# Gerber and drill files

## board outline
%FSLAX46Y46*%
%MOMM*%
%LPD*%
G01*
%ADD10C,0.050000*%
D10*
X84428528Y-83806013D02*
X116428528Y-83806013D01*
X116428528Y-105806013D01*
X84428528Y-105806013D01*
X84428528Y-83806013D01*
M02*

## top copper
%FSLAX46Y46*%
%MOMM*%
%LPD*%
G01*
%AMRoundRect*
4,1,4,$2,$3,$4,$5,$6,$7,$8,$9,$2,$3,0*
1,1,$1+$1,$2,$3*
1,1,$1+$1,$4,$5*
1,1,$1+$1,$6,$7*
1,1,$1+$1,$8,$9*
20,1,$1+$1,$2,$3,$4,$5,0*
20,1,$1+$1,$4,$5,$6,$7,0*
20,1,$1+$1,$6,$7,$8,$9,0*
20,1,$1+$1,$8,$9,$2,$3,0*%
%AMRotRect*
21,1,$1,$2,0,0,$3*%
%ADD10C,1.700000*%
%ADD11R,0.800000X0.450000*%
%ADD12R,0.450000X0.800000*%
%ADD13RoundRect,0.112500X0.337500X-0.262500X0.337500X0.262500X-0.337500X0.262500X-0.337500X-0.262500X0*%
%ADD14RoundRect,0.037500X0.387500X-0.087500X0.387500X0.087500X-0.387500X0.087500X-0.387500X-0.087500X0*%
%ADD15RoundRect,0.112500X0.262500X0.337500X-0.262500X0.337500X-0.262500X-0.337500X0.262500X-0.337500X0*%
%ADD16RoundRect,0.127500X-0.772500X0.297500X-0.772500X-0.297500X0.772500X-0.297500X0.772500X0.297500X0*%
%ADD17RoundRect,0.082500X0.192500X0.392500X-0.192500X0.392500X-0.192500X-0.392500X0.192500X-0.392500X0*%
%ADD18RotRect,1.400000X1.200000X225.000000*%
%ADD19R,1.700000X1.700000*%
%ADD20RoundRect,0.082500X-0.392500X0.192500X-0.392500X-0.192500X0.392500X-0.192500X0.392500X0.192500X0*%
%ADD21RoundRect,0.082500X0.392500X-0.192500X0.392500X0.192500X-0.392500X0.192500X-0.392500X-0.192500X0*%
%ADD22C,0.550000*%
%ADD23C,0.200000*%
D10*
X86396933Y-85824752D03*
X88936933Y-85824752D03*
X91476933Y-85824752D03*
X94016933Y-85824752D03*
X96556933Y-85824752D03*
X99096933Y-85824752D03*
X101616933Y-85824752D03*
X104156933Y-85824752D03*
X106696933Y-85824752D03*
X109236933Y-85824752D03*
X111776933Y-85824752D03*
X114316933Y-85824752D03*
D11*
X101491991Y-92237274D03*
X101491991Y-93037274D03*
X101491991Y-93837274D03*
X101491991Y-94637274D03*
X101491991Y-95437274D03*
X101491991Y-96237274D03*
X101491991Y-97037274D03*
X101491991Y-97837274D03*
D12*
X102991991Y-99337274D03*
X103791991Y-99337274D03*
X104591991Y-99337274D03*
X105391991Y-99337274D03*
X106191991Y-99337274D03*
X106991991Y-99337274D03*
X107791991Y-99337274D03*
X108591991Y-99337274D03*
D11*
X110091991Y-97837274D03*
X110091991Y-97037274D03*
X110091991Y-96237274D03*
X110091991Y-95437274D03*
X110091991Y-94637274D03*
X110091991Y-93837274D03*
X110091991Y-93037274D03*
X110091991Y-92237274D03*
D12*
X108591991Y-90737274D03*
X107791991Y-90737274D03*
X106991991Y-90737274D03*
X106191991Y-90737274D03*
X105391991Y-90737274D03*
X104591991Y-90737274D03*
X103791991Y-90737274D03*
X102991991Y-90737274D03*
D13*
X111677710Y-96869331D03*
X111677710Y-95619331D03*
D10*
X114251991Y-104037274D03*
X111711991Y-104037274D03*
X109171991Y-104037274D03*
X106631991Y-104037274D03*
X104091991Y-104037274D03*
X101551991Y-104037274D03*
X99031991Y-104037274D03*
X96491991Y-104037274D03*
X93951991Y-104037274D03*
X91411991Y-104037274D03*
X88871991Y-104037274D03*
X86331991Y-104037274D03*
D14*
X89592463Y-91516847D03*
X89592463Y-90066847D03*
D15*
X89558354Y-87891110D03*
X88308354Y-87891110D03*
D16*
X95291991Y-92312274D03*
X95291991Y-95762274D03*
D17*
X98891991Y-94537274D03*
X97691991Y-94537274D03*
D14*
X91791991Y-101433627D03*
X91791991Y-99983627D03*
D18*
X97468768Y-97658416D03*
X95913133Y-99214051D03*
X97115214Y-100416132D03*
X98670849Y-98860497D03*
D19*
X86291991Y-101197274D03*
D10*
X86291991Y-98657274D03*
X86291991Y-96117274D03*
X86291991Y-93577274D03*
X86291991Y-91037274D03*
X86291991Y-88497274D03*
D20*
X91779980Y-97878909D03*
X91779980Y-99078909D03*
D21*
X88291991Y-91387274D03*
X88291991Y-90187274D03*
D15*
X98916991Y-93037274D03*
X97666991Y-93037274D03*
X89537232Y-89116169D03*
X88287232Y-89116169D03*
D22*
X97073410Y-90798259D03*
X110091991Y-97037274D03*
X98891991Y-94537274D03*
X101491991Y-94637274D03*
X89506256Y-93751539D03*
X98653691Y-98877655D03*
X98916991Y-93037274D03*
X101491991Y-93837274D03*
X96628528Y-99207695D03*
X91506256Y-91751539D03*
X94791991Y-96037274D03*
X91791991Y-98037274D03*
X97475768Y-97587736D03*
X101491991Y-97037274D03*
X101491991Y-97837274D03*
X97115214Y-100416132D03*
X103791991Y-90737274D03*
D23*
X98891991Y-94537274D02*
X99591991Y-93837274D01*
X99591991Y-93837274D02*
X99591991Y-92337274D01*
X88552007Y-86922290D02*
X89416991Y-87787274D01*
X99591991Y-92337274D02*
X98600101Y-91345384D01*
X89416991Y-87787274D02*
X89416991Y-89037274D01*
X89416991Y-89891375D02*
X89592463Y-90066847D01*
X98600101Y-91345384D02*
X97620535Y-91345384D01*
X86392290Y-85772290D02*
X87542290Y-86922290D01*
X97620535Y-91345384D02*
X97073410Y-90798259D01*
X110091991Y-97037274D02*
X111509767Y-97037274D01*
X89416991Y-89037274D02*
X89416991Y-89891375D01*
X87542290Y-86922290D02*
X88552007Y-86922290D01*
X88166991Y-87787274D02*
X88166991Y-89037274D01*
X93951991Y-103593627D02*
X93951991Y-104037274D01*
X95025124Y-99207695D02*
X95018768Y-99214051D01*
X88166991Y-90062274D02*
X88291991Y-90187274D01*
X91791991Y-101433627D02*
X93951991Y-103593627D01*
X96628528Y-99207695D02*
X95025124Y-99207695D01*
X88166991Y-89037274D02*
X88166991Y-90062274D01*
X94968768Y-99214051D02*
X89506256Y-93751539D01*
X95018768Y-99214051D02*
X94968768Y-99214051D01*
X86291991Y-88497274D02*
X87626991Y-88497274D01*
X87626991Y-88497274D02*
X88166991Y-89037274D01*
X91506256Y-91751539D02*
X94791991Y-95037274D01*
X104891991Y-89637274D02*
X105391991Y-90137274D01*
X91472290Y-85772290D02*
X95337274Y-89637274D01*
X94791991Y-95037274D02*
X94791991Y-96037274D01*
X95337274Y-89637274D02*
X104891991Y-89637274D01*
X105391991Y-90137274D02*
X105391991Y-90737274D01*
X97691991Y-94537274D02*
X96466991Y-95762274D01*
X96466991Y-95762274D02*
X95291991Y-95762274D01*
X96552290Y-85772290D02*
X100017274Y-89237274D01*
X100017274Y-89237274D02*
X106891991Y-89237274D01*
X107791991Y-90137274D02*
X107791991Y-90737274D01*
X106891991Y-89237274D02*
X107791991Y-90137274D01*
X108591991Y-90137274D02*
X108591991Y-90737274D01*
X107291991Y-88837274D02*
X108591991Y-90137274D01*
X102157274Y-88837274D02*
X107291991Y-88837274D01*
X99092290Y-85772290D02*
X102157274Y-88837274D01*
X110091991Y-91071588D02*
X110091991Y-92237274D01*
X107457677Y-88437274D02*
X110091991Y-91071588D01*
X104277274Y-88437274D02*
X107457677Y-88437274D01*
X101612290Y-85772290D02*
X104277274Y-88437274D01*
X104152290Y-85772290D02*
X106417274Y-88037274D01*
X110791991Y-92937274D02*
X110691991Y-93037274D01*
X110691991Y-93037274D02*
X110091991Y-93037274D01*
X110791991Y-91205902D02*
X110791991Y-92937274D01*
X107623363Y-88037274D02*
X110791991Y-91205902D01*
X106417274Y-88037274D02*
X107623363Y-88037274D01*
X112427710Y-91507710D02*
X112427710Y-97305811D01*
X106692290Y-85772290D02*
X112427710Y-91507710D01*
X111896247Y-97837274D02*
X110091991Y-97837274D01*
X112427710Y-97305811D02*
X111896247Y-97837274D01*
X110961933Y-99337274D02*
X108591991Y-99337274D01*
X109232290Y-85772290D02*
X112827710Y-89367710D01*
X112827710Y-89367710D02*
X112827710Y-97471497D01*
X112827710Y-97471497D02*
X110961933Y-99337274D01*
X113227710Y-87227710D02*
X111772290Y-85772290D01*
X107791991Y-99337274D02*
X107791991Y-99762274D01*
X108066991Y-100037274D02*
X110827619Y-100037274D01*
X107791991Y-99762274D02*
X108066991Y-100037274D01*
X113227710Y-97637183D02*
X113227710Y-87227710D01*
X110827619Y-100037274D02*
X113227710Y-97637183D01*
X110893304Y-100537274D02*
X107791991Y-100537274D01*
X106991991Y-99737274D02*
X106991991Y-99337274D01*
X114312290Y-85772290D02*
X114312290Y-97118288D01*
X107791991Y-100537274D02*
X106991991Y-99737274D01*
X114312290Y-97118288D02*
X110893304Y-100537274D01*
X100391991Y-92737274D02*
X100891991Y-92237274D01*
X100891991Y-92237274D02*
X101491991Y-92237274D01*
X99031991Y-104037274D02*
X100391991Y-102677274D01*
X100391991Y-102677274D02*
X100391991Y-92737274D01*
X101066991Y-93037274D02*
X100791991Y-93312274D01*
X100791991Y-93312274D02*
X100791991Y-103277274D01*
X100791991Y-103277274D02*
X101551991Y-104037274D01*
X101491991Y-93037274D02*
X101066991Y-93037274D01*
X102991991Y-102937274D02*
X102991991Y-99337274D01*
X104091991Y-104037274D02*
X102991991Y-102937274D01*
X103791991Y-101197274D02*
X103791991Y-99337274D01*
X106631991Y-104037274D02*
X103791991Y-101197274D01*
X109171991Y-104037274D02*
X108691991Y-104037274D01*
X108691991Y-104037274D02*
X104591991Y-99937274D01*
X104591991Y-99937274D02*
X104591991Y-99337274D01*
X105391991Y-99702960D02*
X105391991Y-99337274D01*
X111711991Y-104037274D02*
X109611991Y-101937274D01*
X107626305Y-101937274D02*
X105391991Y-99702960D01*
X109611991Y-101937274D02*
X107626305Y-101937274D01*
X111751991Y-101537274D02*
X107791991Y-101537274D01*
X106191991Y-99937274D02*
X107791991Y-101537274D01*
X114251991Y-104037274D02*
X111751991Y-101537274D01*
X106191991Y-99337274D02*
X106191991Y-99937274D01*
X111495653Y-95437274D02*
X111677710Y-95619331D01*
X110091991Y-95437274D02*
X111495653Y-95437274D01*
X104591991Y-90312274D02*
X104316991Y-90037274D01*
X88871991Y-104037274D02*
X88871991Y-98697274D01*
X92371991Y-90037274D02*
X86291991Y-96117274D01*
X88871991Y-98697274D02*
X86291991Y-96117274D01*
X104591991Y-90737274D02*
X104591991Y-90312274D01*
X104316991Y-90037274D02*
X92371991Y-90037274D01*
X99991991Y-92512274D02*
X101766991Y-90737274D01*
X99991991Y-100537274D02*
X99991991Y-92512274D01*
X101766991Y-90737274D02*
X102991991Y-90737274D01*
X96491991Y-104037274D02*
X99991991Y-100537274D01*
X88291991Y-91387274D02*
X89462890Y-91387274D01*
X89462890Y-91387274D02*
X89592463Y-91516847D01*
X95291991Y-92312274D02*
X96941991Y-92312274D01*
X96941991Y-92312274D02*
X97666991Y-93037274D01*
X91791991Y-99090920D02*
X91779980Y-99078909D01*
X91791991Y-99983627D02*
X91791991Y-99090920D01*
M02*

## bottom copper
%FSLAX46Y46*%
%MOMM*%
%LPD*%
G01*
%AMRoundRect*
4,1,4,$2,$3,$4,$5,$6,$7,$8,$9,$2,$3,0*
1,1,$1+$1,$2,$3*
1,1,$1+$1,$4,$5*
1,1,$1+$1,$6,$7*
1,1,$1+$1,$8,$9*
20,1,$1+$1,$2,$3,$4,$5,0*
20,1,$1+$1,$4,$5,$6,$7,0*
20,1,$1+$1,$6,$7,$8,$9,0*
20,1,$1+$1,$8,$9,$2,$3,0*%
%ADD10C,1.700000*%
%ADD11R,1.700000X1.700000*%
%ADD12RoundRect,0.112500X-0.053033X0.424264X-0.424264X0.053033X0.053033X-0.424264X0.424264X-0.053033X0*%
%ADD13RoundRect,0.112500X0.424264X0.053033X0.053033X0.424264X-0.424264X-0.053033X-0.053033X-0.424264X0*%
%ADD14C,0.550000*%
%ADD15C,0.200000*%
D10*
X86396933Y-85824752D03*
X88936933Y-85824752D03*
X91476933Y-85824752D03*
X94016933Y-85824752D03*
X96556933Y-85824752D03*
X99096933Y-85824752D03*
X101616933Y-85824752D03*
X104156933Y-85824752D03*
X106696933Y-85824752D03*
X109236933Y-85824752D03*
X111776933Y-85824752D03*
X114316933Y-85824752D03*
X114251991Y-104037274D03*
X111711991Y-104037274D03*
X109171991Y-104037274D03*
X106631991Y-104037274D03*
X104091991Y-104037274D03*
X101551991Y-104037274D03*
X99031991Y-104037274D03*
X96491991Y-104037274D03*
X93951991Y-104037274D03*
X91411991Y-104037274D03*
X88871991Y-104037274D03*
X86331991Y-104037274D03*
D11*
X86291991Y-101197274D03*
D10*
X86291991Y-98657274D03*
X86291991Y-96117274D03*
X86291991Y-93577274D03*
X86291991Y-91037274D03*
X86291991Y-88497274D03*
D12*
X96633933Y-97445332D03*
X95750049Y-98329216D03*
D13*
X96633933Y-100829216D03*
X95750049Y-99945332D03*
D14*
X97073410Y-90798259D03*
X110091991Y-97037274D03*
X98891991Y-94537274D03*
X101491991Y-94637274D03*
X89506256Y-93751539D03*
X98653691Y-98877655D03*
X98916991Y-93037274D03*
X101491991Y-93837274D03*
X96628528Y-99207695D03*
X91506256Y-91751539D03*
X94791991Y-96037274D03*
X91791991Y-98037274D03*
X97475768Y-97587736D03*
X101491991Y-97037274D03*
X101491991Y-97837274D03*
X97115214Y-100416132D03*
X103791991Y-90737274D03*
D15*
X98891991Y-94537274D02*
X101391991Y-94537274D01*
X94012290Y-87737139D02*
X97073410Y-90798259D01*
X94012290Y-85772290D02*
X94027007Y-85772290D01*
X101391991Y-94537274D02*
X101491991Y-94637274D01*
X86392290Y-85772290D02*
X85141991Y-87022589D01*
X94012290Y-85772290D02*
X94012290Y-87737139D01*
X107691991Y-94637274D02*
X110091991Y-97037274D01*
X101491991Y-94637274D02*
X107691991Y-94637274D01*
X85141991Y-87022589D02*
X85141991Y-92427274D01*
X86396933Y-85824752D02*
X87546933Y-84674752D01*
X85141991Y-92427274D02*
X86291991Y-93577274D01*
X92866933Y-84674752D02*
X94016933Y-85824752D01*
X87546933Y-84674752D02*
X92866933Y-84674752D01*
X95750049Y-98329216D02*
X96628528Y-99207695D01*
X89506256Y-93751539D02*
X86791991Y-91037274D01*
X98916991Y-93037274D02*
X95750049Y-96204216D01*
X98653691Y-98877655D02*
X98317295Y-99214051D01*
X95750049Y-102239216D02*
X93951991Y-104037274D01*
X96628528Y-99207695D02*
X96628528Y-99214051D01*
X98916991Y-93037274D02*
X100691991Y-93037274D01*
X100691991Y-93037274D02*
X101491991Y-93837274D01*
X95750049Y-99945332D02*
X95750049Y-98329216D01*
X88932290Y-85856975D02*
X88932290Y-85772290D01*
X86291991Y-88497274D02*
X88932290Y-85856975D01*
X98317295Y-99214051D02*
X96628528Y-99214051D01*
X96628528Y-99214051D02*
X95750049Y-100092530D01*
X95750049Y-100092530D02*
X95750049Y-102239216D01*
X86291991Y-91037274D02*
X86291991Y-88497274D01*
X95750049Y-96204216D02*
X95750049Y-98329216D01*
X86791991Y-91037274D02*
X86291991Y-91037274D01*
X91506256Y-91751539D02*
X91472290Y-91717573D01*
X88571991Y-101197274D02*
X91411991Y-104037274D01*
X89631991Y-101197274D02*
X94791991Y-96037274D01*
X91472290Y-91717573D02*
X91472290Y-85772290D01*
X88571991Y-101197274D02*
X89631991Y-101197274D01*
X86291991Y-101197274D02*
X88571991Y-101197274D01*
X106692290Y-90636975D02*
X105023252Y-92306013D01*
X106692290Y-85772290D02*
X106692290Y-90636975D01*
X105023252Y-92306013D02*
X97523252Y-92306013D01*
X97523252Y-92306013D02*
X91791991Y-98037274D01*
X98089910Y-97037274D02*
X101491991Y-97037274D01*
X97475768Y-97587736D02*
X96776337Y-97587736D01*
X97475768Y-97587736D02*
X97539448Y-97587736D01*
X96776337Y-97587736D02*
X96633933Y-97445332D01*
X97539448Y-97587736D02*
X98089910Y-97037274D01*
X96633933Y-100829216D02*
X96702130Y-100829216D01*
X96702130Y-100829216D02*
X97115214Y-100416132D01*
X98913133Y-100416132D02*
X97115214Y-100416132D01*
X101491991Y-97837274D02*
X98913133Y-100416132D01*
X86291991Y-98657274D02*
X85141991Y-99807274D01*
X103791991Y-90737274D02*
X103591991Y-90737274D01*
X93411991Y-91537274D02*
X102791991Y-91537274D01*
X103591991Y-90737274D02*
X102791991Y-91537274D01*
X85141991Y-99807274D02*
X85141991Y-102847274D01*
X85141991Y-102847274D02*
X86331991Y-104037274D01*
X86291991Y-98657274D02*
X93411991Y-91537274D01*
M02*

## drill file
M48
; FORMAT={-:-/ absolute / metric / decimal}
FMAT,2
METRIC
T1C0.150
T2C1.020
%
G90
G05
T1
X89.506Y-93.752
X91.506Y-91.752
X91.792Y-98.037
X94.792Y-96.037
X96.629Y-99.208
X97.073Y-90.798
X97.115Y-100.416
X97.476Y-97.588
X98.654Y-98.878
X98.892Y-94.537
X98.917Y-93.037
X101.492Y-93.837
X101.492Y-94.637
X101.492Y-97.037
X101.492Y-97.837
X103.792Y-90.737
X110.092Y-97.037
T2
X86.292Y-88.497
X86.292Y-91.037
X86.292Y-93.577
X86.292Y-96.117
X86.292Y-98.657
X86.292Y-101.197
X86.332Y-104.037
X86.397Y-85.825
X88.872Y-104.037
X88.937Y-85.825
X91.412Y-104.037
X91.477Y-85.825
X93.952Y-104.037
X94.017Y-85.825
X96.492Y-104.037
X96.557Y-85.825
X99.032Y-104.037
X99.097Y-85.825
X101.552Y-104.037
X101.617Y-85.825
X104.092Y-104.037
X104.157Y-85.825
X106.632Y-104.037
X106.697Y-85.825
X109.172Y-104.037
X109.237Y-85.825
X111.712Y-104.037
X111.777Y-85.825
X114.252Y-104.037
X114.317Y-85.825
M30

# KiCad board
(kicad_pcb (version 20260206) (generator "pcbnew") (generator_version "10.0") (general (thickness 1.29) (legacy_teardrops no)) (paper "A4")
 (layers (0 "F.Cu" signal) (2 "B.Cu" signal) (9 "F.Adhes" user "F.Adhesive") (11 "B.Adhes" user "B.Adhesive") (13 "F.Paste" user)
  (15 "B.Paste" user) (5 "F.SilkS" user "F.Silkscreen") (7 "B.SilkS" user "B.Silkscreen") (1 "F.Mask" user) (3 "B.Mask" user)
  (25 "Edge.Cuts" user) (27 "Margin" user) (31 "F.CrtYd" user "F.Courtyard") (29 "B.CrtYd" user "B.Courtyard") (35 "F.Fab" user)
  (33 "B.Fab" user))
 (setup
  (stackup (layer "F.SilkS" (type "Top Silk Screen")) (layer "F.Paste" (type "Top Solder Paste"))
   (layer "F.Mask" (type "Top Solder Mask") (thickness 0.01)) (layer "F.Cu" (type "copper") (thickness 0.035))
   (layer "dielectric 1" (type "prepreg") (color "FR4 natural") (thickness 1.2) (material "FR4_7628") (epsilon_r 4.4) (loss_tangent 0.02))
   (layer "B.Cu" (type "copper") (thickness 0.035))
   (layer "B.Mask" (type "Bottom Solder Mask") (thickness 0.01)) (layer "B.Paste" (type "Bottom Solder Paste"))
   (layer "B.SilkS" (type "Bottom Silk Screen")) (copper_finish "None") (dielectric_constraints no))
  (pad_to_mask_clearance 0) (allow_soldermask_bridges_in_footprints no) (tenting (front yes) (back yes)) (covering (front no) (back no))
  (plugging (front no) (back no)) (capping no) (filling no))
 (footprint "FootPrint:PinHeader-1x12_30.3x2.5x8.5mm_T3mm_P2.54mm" (layer "F.Cu") (at 100.356933 85.824752)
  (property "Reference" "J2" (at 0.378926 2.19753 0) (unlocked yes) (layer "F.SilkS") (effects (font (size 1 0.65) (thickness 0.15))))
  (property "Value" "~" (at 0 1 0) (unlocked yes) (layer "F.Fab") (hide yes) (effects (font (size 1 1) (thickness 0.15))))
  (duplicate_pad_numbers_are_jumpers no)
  (pad "1" thru_hole circle (at -13.96 0) (size 1.7 1.7) (drill 1.02) (layers "*.Cu" "*.Mask") (remove_unused_layers no) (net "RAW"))
  (pad "2" thru_hole circle (at -11.42 0) (size 1.7 1.7) (drill 1.02) (layers "*.Cu" "*.Mask") (remove_unused_layers no) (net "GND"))
  (pad "3" thru_hole circle (at -8.88 0) (size 1.7 1.7) (drill 1.02) (layers "*.Cu" "*.Mask") (remove_unused_layers no) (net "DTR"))
  (pad "4" thru_hole circle (at -6.34 0) (size 1.7 1.7) (drill 1.02) (layers "*.Cu" "*.Mask") (remove_unused_layers no) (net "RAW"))
  (pad "5" thru_hole circle (at -3.8 0) (size 1.7 1.7) (drill 1.02) (layers "*.Cu" "*.Mask") (remove_unused_layers no) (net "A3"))
  (pad "6" thru_hole circle (at -1.26 0) (size 1.7 1.7) (drill 1.02) (layers "*.Cu" "*.Mask") (remove_unused_layers no) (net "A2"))
  (pad "7" thru_hole circle (at 1.26 0) (size 1.7 1.7) (drill 1.02) (layers "*.Cu" "*.Mask") (remove_unused_layers no) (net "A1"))
  (pad "8" thru_hole circle (at 3.8 0) (size 1.7 1.7) (drill 1.02) (layers "*.Cu" "*.Mask") (remove_unused_layers no) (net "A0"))
  (pad "9" thru_hole circle (at 6.34 0) (size 1.7 1.7) (drill 1.02) (layers "*.Cu" "*.Mask") (remove_unused_layers no) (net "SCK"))
  (pad "10" thru_hole circle (at 8.88 0) (size 1.7 1.7) (drill 1.02) (layers "*.Cu" "*.Mask") (remove_unused_layers no) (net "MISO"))
  (pad "11" thru_hole circle (at 11.42 0) (size 1.7 1.7) (drill 1.02) (layers "*.Cu" "*.Mask") (remove_unused_layers no) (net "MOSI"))
  (pad "12" thru_hole circle (at 13.96 0) (size 1.7 1.7) (drill 1.02) (layers "*.Cu" "*.Mask") (remove_unused_layers no) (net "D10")))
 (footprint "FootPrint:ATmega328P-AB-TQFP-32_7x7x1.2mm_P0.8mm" (layer "F.Cu") (at 105.791991 95.037274)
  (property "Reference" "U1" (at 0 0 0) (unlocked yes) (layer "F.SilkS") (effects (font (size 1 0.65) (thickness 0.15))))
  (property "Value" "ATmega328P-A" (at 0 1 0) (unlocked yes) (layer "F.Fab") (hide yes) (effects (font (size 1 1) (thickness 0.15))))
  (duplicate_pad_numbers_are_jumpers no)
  (pad "1" smd rect (at -4.3 -2.8) (size 0.8 0.45) (layers "F.Cu" "F.Mask" "F.Paste") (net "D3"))
  (pad "2" smd rect (at -4.3 -2) (size 0.8 0.45) (layers "F.Cu" "F.Mask" "F.Paste") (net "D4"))
  (pad "3" smd rect (at -4.3 -1.2) (size 0.8 0.45) (layers "F.Cu" "F.Mask" "F.Paste") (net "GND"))
  (pad "4" smd rect (at -4.3 -0.4) (size 0.8 0.45) (layers "F.Cu" "F.Mask" "F.Paste") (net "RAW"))
  (pad "5" smd rect (at -4.3 0.4) (size 0.8 0.45) (layers "F.Cu" "F.Mask" "F.Paste") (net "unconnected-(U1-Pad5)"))
  (pad "6" smd rect (at -4.3 1.2) (size 0.8 0.45) (layers "F.Cu" "F.Mask" "F.Paste") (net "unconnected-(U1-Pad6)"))
  (pad "7" smd rect (at -4.3 2) (size 0.8 0.45) (layers "F.Cu" "F.Mask" "F.Paste") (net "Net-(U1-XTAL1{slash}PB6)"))
  (pad "8" smd rect (at -4.3 2.8) (size 0.8 0.45) (layers "F.Cu" "F.Mask" "F.Paste") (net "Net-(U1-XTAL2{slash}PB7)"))
  (pad "9" smd rect (at -2.8 4.3 90) (size 0.8 0.45) (layers "F.Cu" "F.Mask" "F.Paste") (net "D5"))
  (pad "10" smd rect (at -2 4.3 90) (size 0.8 0.45) (layers "F.Cu" "F.Mask" "F.Paste") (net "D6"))
  (pad "11" smd rect (at -1.2 4.3 90) (size 0.8 0.45) (layers "F.Cu" "F.Mask" "F.Paste") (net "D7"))
  (pad "12" smd rect (at -0.4 4.3 90) (size 0.8 0.45) (layers "F.Cu" "F.Mask" "F.Paste") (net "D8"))
  (pad "13" smd rect (at 0.4 4.3 90) (size 0.8 0.45) (layers "F.Cu" "F.Mask" "F.Paste") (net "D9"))
  (pad "14" smd rect (at 1.2 4.3 90) (size 0.8 0.45) (layers "F.Cu" "F.Mask" "F.Paste") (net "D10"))
  (pad "15" smd rect (at 2 4.3 90) (size 0.8 0.45) (layers "F.Cu" "F.Mask" "F.Paste") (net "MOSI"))
  (pad "16" smd rect (at 2.8 4.3 90) (size 0.8 0.45) (layers "F.Cu" "F.Mask" "F.Paste") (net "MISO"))
  (pad "17" smd rect (at 4.3 2.8) (size 0.8 0.45) (layers "F.Cu" "F.Mask" "F.Paste") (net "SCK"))
  (pad "18" smd rect (at 4.3 2) (size 0.8 0.45) (layers "F.Cu" "F.Mask" "F.Paste") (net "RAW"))
  (pad "19" smd rect (at 4.3 1.2) (size 0.8 0.45) (layers "F.Cu" "F.Mask" "F.Paste") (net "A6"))
  (pad "20" smd rect (at 4.3 0.4) (size 0.8 0.45) (layers "F.Cu" "F.Mask" "F.Paste") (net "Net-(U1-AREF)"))
  (pad "21" smd rect (at 4.3 -0.4) (size 0.8 0.45) (layers "F.Cu" "F.Mask" "F.Paste") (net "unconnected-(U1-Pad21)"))
  (pad "22" smd rect (at 4.3 -1.2) (size 0.8 0.45) (layers "F.Cu" "F.Mask" "F.Paste") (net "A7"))
  (pad "23" smd rect (at 4.3 -2) (size 0.8 0.45) (layers "F.Cu" "F.Mask" "F.Paste") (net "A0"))
  (pad "24" smd rect (at 4.3 -2.8) (size 0.8 0.45) (layers "F.Cu" "F.Mask" "F.Paste") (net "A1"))
  (pad "25" smd rect (at 2.8 -4.3 90) (size 0.8 0.45) (layers "F.Cu" "F.Mask" "F.Paste") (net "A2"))
  (pad "26" smd rect (at 2 -4.3 90) (size 0.8 0.45) (layers "F.Cu" "F.Mask" "F.Paste") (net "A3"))
  (pad "27" smd rect (at 1.2 -4.3 90) (size 0.8 0.45) (layers "F.Cu" "F.Mask" "F.Paste") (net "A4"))
  (pad "28" smd rect (at 0.4 -4.3 90) (size 0.8 0.45) (layers "F.Cu" "F.Mask" "F.Paste") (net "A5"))
  (pad "29" smd rect (at -0.4 -4.3 90) (size 0.8 0.45) (layers "F.Cu" "F.Mask" "F.Paste") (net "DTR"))
  (pad "30" smd rect (at -1.2 -4.3 90) (size 0.8 0.45) (layers "F.Cu" "F.Mask" "F.Paste") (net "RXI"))
  (pad "31" smd rect (at -2 -4.3 90) (size 0.8 0.45) (layers "F.Cu" "F.Mask" "F.Paste") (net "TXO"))
  (pad "32" smd rect (at -2.8 -4.3 90) (size 0.8 0.45) (layers "F.Cu" "F.Mask" "F.Paste") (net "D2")))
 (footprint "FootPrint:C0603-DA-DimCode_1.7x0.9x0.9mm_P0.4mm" (layer "F.Cu") (at 111.67771 96.244331 90)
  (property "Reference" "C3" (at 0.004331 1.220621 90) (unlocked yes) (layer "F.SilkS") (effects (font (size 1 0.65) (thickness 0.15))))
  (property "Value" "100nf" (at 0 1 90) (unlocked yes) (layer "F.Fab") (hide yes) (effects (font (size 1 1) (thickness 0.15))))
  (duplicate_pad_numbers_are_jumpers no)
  (pad "1" smd roundrect (at -0.625 0 90) (size 0.75 0.9) (layers "F.Cu" "F.Mask" "F.Paste") (roundrect_rratio 0.15) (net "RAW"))
  (pad "2" smd roundrect (at 0.625 0 90) (size 0.75 0.9) (layers "F.Cu" "F.Mask" "F.Paste") (roundrect_rratio 0.15) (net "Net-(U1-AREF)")))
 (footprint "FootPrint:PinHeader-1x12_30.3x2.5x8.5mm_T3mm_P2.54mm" (layer "F.Cu") (at 100.291991 104.037274 180)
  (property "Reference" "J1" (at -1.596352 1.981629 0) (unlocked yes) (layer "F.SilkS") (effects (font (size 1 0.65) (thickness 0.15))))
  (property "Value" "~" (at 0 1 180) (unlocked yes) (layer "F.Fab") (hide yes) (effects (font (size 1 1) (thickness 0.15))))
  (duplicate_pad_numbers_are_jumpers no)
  (pad "1" thru_hole circle (at -13.96 0 180) (size 1.7 1.7) (drill 1.02) (layers "*.Cu" "*.Mask") (remove_unused_layers no) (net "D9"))
  (pad "2" thru_hole circle (at -11.42 0 180) (size 1.7 1.7) (drill 1.02) (layers "*.Cu" "*.Mask") (remove_unused_layers no) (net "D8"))
  (pad "3" thru_hole circle (at -8.88 0 180) (size 1.7 1.7) (drill 1.02) (layers "*.Cu" "*.Mask") (remove_unused_layers no) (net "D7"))
  (pad "4" thru_hole circle (at -6.34 0 180) (size 1.7 1.7) (drill 1.02) (layers "*.Cu" "*.Mask") (remove_unused_layers no) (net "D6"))
  (pad "5" thru_hole circle (at -3.8 0 180) (size 1.7 1.7) (drill 1.02) (layers "*.Cu" "*.Mask") (remove_unused_layers no) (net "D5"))
  (pad "6" thru_hole circle (at -1.26 0 180) (size 1.7 1.7) (drill 1.02) (layers "*.Cu" "*.Mask") (remove_unused_layers no) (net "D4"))
  (pad "7" thru_hole circle (at 1.26 0 180) (size 1.7 1.7) (drill 1.02) (layers "*.Cu" "*.Mask") (remove_unused_layers no) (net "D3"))
  (pad "8" thru_hole circle (at 3.8 0 180) (size 1.7 1.7) (drill 1.02) (layers "*.Cu" "*.Mask") (remove_unused_layers no) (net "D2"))
  (pad "9" thru_hole circle (at 6.34 0 180) (size 1.7 1.7) (drill 1.02) (layers "*.Cu" "*.Mask") (remove_unused_layers no) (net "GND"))
  (pad "10" thru_hole circle (at 8.88 0 180) (size 1.7 1.7) (drill 1.02) (layers "*.Cu" "*.Mask") (remove_unused_layers no) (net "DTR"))
  (pad "11" thru_hole circle (at 11.42 0 180) (size 1.7 1.7) (drill 1.02) (layers "*.Cu" "*.Mask") (remove_unused_layers no) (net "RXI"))
  (pad "12" thru_hole circle (at 13.96 0 180) (size 1.7 1.7) (drill 1.02) (layers "*.Cu" "*.Mask") (remove_unused_layers no) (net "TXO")))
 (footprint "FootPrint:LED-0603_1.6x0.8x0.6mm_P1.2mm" (layer "F.Cu") (at 89.592463 90.791847 90)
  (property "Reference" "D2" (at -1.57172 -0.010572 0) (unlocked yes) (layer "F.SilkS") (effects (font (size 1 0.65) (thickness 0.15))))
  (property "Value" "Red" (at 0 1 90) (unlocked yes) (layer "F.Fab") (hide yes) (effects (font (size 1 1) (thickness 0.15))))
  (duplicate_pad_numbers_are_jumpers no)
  (pad "1" smd roundrect (at -0.725 0 90) (size 0.25 0.85) (layers "F.Cu" "F.Mask" "F.Paste") (roundrect_rratio 0.15) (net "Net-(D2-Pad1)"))
  (pad "2" smd roundrect (at 0.725 0 90) (size 0.25 0.85) (layers "F.Cu" "F.Mask" "F.Paste") (roundrect_rratio 0.15) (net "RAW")))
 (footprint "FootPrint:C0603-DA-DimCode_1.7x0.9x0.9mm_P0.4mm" (layer "F.Cu") (at 88.933354 87.89111 180)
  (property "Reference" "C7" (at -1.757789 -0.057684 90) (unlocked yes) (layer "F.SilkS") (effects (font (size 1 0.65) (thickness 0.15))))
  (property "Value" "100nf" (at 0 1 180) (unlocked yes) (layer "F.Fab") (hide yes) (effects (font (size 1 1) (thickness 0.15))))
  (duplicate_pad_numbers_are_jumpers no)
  (pad "1" smd roundrect (at -0.625 0 180) (size 0.75 0.9) (layers "F.Cu" "F.Mask" "F.Paste") (roundrect_rratio 0.15) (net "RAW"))
  (pad "2" smd roundrect (at 0.625 0 180) (size 0.75 0.9) (layers "F.Cu" "F.Mask" "F.Paste") (roundrect_rratio 0.15) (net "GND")))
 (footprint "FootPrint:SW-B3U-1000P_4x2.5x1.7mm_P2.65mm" (layer "F.Cu") (at 95.291991 94.037274 -90)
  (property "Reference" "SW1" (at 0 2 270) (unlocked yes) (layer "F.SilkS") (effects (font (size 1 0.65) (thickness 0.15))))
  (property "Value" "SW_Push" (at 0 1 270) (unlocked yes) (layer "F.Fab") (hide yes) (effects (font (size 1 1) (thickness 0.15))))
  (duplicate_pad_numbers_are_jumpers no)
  (pad "1" smd roundrect (at -1.725 0 270) (size 0.85 1.8) (layers "F.Cu" "F.Mask" "F.Paste") (roundrect_rratio 0.15) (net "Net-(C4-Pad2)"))
  (pad "2" smd roundrect (at 1.725 0 270) (size 0.85 1.8) (layers "F.Cu" "F.Mask" "F.Paste") (roundrect_rratio 0.15) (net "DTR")))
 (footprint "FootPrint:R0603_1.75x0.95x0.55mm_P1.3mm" (layer "F.Cu") (at 98.291991 94.537274 180)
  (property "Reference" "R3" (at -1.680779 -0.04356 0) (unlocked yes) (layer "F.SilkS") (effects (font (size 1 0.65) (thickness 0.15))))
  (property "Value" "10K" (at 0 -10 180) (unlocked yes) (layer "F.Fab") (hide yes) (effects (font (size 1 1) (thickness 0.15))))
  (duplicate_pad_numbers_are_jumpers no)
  (pad "1" smd roundrect (at -0.6 0 180) (size 0.55 0.95) (layers "F.Cu" "F.Mask" "F.Paste") (roundrect_rratio 0.15) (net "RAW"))
  (pad "2" smd roundrect (at 0.6 0 180) (size 0.55 0.95) (layers "F.Cu" "F.Mask" "F.Paste") (roundrect_rratio 0.15) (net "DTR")))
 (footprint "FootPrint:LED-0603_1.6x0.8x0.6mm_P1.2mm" (layer "F.Cu") (at 91.791991 100.708627 90)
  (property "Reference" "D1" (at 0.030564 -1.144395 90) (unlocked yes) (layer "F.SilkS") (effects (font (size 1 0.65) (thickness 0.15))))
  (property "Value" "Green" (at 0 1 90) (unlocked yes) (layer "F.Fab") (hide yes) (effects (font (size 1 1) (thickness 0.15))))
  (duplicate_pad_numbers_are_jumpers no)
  (pad "1" smd roundrect (at -0.725 0 90) (size 0.25 0.85) (layers "F.Cu" "F.Mask" "F.Paste") (roundrect_rratio 0.15) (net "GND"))
  (pad "2" smd roundrect (at 0.725 0 90) (size 0.25 0.85) (layers "F.Cu" "F.Mask" "F.Paste") (roundrect_rratio 0.15) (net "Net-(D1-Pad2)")))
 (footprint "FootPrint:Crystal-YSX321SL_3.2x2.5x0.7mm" (layer "F.Cu") (at 97.291991 99.037274 -135)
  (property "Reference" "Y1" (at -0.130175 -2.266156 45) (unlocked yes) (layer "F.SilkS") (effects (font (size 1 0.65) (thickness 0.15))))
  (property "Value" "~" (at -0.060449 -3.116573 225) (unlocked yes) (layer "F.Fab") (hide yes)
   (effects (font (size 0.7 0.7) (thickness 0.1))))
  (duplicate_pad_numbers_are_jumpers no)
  (pad "1" smd rect (at -1.1 0.85 225) (size 1.4 1.2) (layers "F.Cu" "F.Mask" "F.Paste") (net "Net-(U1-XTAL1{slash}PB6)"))
  (pad "2" smd rect (at 1.1 0.85 225) (size 1.4 1.2) (layers "F.Cu" "F.Mask" "F.Paste") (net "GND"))
  (pad "3" smd rect (at 1.1 -0.85 225) (size 1.4 1.2) (layers "F.Cu" "F.Mask" "F.Paste") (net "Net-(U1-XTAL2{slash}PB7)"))
  (pad "4" smd rect (at -1.1 -0.85 225) (size 1.4 1.2) (layers "F.Cu" "F.Mask" "F.Paste") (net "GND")))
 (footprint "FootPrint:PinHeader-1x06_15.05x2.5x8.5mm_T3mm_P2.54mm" (layer "F.Cu") (at 86.291991 94.847274 90)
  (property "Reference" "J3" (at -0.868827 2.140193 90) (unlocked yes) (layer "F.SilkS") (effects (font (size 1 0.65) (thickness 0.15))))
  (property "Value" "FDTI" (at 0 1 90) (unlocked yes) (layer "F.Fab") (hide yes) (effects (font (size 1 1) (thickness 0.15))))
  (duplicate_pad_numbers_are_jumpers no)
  (pad "1" thru_hole rect (at -6.35 0 90) (size 1.7 1.7) (drill 1.02) (layers "*.Cu" "*.Mask") (remove_unused_layers no) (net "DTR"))
  (pad "2" thru_hole circle (at -3.81 0 90) (size 1.7 1.7) (drill 1.02) (layers "*.Cu" "*.Mask") (remove_unused_layers no) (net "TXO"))
  (pad "3" thru_hole circle (at -1.27 0 90) (size 1.7 1.7) (drill 1.02) (layers "*.Cu" "*.Mask") (remove_unused_layers no) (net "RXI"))
  (pad "4" thru_hole circle (at 1.27 0 90) (size 1.7 1.7) (drill 1.02) (layers "*.Cu" "*.Mask") (remove_unused_layers no) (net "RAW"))
  (pad "5" thru_hole circle (at 3.81 0 90) (size 1.7 1.7) (drill 1.02) (layers "*.Cu" "*.Mask") (remove_unused_layers no) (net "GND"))
  (pad "6" thru_hole circle (at 6.35 0 90) (size 1.7 1.7) (drill 1.02) (layers "*.Cu" "*.Mask") (remove_unused_layers no) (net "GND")))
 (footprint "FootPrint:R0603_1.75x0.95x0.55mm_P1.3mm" (layer "F.Cu") (at 91.77998 98.478909 -90)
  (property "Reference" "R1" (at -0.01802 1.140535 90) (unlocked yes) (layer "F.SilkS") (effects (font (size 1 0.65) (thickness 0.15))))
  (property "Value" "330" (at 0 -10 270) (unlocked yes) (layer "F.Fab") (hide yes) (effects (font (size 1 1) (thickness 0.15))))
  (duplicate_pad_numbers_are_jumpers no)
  (pad "1" smd roundrect (at -0.6 0 270) (size 0.55 0.95) (layers "F.Cu" "F.Mask" "F.Paste") (roundrect_rratio 0.15) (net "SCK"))
  (pad "2" smd roundrect (at 0.6 0 270) (size 0.55 0.95) (layers "F.Cu" "F.Mask" "F.Paste") (roundrect_rratio 0.15) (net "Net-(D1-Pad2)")))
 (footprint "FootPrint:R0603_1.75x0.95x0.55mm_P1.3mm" (layer "F.Cu") (at 88.291991 90.787274 90)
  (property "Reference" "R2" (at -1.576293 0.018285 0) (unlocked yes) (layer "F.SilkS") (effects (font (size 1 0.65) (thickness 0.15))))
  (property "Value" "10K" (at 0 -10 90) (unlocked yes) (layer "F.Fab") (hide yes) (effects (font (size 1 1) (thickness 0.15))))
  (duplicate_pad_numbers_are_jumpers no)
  (pad "1" smd roundrect (at -0.6 0 90) (size 0.55 0.95) (layers "F.Cu" "F.Mask" "F.Paste") (roundrect_rratio 0.15) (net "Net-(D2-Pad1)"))
  (pad "2" smd roundrect (at 0.6 0 90) (size 0.55 0.95) (layers "F.Cu" "F.Mask" "F.Paste") (roundrect_rratio 0.15) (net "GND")))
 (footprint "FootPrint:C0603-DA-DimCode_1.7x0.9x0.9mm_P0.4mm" (layer "F.Cu") (at 98.291991 93.037274 180)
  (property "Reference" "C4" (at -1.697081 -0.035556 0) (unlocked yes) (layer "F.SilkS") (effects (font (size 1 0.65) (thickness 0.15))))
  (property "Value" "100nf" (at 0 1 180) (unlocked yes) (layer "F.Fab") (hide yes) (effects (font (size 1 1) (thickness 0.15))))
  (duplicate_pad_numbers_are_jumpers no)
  (pad "1" smd roundrect (at -0.625 0 180) (size 0.75 0.9) (layers "F.Cu" "F.Mask" "F.Paste") (roundrect_rratio 0.15) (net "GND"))
  (pad "2" smd roundrect (at 0.625 0 180) (size 0.75 0.9) (layers "F.Cu" "F.Mask" "F.Paste") (roundrect_rratio 0.15) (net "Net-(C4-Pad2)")))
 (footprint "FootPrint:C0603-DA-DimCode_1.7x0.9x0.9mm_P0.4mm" (layer "F.Cu") (at 88.912232 89.116169 180)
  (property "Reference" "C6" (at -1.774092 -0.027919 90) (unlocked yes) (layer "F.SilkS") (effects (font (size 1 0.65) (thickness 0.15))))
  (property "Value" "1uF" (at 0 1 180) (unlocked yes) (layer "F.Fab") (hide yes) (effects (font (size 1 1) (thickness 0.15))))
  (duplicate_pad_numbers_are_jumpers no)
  (pad "1" smd roundrect (at -0.625 0 180) (size 0.75 0.9) (layers "F.Cu" "F.Mask" "F.Paste") (roundrect_rratio 0.15) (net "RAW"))
  (pad "2" smd roundrect (at 0.625 0 180) (size 0.75 0.9) (layers "F.Cu" "F.Mask" "F.Paste") (roundrect_rratio 0.15) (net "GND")))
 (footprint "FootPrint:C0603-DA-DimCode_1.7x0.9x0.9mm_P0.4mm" (layer "B.Cu") (at 96.191991 97.887274 -135)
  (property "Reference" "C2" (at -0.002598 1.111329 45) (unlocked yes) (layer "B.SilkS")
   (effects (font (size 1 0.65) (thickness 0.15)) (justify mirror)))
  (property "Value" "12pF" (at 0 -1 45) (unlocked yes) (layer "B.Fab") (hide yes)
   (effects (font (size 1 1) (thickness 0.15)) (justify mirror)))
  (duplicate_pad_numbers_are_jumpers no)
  (pad "1" smd roundrect (at -0.625 0 225) (size 0.75 0.9) (layers "B.Cu" "B.Mask" "B.Paste") (roundrect_rratio 0.15)
   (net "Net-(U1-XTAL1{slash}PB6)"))
  (pad "2" smd roundrect (at 0.625 0 225) (size 0.75 0.9) (layers "B.Cu" "B.Mask" "B.Paste") (roundrect_rratio 0.15) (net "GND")))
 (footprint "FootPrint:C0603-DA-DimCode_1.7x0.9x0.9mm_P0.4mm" (layer "B.Cu") (at 96.191991 100.387274 135)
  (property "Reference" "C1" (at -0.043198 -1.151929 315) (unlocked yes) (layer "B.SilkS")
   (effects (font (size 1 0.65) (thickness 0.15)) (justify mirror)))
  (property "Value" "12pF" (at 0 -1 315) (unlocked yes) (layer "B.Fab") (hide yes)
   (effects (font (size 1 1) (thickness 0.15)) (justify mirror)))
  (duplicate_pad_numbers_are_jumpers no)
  (pad "1" smd roundrect (at -0.625 0 135) (size 0.75 0.9) (layers "B.Cu" "B.Mask" "B.Paste") (roundrect_rratio 0.15)
   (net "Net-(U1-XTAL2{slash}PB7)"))
  (pad "2" smd roundrect (at 0.625 0 135) (size 0.75 0.9) (layers "B.Cu" "B.Mask" "B.Paste") (roundrect_rratio 0.15) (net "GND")))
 (gr_rect (start 84.428528 83.806013) (end 116.428528 105.806013) (stroke (width 0.05) (type solid)) (fill no) (layer "Edge.Cuts"))
 (segment (start 98.891991 94.537274) (end 99.591991 93.837274) (width 0.2) (layer "F.Cu") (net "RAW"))
 (segment (start 99.591991 93.837274) (end 99.591991 92.337274) (width 0.2) (layer "F.Cu") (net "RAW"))
 (segment (start 88.552007 86.92229) (end 89.416991 87.787274) (width 0.2) (layer "F.Cu") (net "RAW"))
 (segment (start 99.591991 92.337274) (end 98.600101 91.345384) (width 0.2) (layer "F.Cu") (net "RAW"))
 (segment (start 89.416991 87.787274) (end 89.416991 89.037274) (width 0.2) (layer "F.Cu") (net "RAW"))
 (segment (start 89.416991 89.891375) (end 89.592463 90.066847) (width 0.2) (layer "F.Cu") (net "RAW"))
 (segment (start 98.600101 91.345384) (end 97.620535 91.345384) (width 0.2) (layer "F.Cu") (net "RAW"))
 (segment (start 86.39229 85.77229) (end 87.54229 86.92229) (width 0.2) (layer "F.Cu") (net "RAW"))
 (segment (start 97.620535 91.345384) (end 97.07341 90.798259) (width 0.2) (layer "F.Cu") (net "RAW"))
 (segment (start 110.091991 97.037274) (end 111.509767 97.037274) (width 0.2) (layer "F.Cu") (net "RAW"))
 (segment (start 89.416991 89.037274) (end 89.416991 89.891375) (width 0.2) (layer "F.Cu") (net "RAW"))
 (segment (start 87.54229 86.92229) (end 88.552007 86.92229) (width 0.2) (layer "F.Cu") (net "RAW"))
 (via (at 97.07341 90.798259) (size 0.55) (drill 0.15) (layers "F.Cu" "B.Cu") (capping no) (covering (front no) (back no))
  (plugging (front no) (back no)) (filling no) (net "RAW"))
 (via (at 110.091991 97.037274) (size 0.55) (drill 0.15) (layers "F.Cu" "B.Cu") (capping no) (covering (front no) (back no))
  (plugging (front no) (back no)) (filling no) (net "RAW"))
 (via (at 98.891991 94.537274) (size 0.55) (drill 0.15) (layers "F.Cu" "B.Cu") (capping no) (covering (front no) (back no))
  (plugging (front no) (back no)) (filling no) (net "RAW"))
 (via (at 101.491991 94.637274) (size 0.55) (drill 0.15) (layers "F.Cu" "B.Cu") (capping no) (covering (front no) (back no))
  (plugging (front no) (back no)) (filling no) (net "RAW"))
 (segment (start 98.891991 94.537274) (end 101.391991 94.537274) (width 0.2) (layer "B.Cu") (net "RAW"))
 (segment (start 94.01229 87.737139) (end 97.07341 90.798259) (width 0.2) (layer "B.Cu") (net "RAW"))
 (segment (start 94.01229 85.77229) (end 94.027007 85.77229) (width 0.2) (layer "B.Cu") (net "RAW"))
 (segment (start 101.391991 94.537274) (end 101.491991 94.637274) (width 0.2) (layer "B.Cu") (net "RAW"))
 (segment (start 86.39229 85.77229) (end 85.141991 87.022589) (width 0.2) (layer "B.Cu") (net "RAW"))
 (segment (start 94.01229 85.77229) (end 94.01229 87.737139) (width 0.2) (layer "B.Cu") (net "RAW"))
 (segment (start 107.691991 94.637274) (end 110.091991 97.037274) (width 0.2) (layer "B.Cu") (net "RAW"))
 (segment (start 101.491991 94.637274) (end 107.691991 94.637274) (width 0.2) (layer "B.Cu") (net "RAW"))
 (segment (start 85.141991 87.022589) (end 85.141991 92.427274) (width 0.2) (layer "B.Cu") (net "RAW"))
 (segment (start 86.396933 85.824752) (end 87.546933 84.674752) (width 0.2) (layer "B.Cu") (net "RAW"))
 (segment (start 85.141991 92.427274) (end 86.291991 93.577274) (width 0.2) (layer "B.Cu") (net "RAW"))
 (segment (start 92.866933 84.674752) (end 94.016933 85.824752) (width 0.2) (layer "B.Cu") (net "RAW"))
 (segment (start 87.546933 84.674752) (end 92.866933 84.674752) (width 0.2) (layer "B.Cu") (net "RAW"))
 (segment (start 88.166991 87.787274) (end 88.166991 89.037274) (width 0.2) (layer "F.Cu") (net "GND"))
 (segment (start 93.951991 103.593627) (end 93.951991 104.037274) (width 0.2) (layer "F.Cu") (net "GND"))
 (segment (start 95.025124 99.207695) (end 95.018768 99.214051) (width 0.2) (layer "F.Cu") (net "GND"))
 (segment (start 88.166991 90.062274) (end 88.291991 90.187274) (width 0.2) (layer "F.Cu") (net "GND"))
 (segment (start 91.791991 101.433627) (end 93.951991 103.593627) (width 0.2) (layer "F.Cu") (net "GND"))
 (segment (start 96.628528 99.207695) (end 95.025124 99.207695) (width 0.2) (layer "F.Cu") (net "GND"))
 (segment (start 88.166991 89.037274) (end 88.166991 90.062274) (width 0.2) (layer "F.Cu") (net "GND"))
 (segment (start 94.968768 99.214051) (end 89.506256 93.751539) (width 0.2) (layer "F.Cu") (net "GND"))
 (segment (start 95.018768 99.214051) (end 94.968768 99.214051) (width 0.2) (layer "F.Cu") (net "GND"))
 (segment (start 86.291991 88.497274) (end 87.626991 88.497274) (width 0.2) (layer "F.Cu") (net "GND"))
 (segment (start 87.626991 88.497274) (end 88.166991 89.037274) (width 0.2) (layer "F.Cu") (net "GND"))
 (via (at 89.506256 93.751539) (size 0.55) (drill 0.15) (layers "F.Cu" "B.Cu") (capping no) (covering (front no) (back no))
  (plugging (front no) (back no)) (filling no) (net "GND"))
 (via (at 98.653691 98.877655) (size 0.55) (drill 0.15) (layers "F.Cu" "B.Cu") (capping no) (covering (front no) (back no))
  (plugging (front no) (back no)) (filling no) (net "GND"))
 (via (at 98.916991 93.037274) (size 0.55) (drill 0.15) (layers "F.Cu" "B.Cu") (capping no) (covering (front no) (back no))
  (plugging (front no) (back no)) (filling no) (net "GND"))
 (via (at 101.491991 93.837274) (size 0.55) (drill 0.15) (layers "F.Cu" "B.Cu") (capping no) (covering (front no) (back no))
  (plugging (front no) (back no)) (filling no) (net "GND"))
 (via (at 96.628528 99.207695) (size 0.55) (drill 0.15) (layers "F.Cu" "B.Cu") (capping no) (covering (front no) (back no))
  (plugging (front no) (back no)) (filling no) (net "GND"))
 (segment (start 95.750049 98.329216) (end 96.628528 99.207695) (width 0.2) (layer "B.Cu") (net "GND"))
 (segment (start 89.506256 93.751539) (end 86.791991 91.037274) (width 0.2) (layer "B.Cu") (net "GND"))
 (segment (start 98.916991 93.037274) (end 95.750049 96.204216) (width 0.2) (layer "B.Cu") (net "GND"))
 (segment (start 98.653691 98.877655) (end 98.317295 99.214051) (width 0.2) (layer "B.Cu") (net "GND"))
 (segment (start 95.750049 102.239216) (end 93.951991 104.037274) (width 0.2) (layer "B.Cu") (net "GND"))
 (segment (start 96.628528 99.207695) (end 96.628528 99.214051) (width 0.2) (layer "B.Cu") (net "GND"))
 (segment (start 98.916991 93.037274) (end 100.691991 93.037274) (width 0.2) (layer "B.Cu") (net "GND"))
 (segment (start 100.691991 93.037274) (end 101.491991 93.837274) (width 0.2) (layer "B.Cu") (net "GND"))
 (segment (start 95.750049 99.945332) (end 95.750049 98.329216) (width 0.2) (layer "B.Cu") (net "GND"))
 (segment (start 88.93229 85.856975) (end 88.93229 85.77229) (width 0.2) (layer "B.Cu") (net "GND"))
 (segment (start 86.291991 88.497274) (end 88.93229 85.856975) (width 0.2) (layer "B.Cu") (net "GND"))
 (segment (start 98.317295 99.214051) (end 96.628528 99.214051) (width 0.2) (layer "B.Cu") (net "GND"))
 (segment (start 96.628528 99.214051) (end 95.750049 100.09253) (width 0.2) (layer "B.Cu") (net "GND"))
 (segment (start 95.750049 100.09253) (end 95.750049 102.239216) (width 0.2) (layer "B.Cu") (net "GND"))
 (segment (start 86.291991 91.037274) (end 86.291991 88.497274) (width 0.2) (layer "B.Cu") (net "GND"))
 (segment (start 95.750049 96.204216) (end 95.750049 98.329216) (width 0.2) (layer "B.Cu") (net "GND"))
 (segment (start 86.791991 91.037274) (end 86.291991 91.037274) (width 0.2) (layer "B.Cu") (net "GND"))
 (segment (start 91.506256 91.751539) (end 94.791991 95.037274) (width 0.2) (layer "F.Cu") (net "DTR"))
 (segment (start 104.891991 89.637274) (end 105.391991 90.137274) (width 0.2) (layer "F.Cu") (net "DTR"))
 (segment (start 91.47229 85.77229) (end 95.337274 89.637274) (width 0.2) (layer "F.Cu") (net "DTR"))
 (segment (start 94.791991 95.037274) (end 94.791991 96.037274) (width 0.2) (layer "F.Cu") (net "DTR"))
 (segment (start 95.337274 89.637274) (end 104.891991 89.637274) (width 0.2) (layer "F.Cu") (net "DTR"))
 (segment (start 105.391991 90.137274) (end 105.391991 90.737274) (width 0.2) (layer "F.Cu") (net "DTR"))
 (segment (start 97.691991 94.537274) (end 96.466991 95.762274) (width 0.2) (layer "F.Cu") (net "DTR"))
 (segment (start 96.466991 95.762274) (end 95.291991 95.762274) (width 0.2) (layer "F.Cu") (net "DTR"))
 (via (at 91.506256 91.751539) (size 0.55) (drill 0.15) (layers "F.Cu" "B.Cu") (capping no) (covering (front no) (back no))
  (plugging (front no) (back no)) (filling no) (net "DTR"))
 (via (at 94.791991 96.037274) (size 0.55) (drill 0.15) (layers "F.Cu" "B.Cu") (capping no) (covering (front no) (back no))
  (plugging (front no) (back no)) (filling no) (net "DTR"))
 (segment (start 91.506256 91.751539) (end 91.47229 91.717573) (width 0.2) (layer "B.Cu") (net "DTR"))
 (segment (start 88.571991 101.197274) (end 91.411991 104.037274) (width 0.2) (layer "B.Cu") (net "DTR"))
 (segment (start 89.631991 101.197274) (end 94.791991 96.037274) (width 0.2) (layer "B.Cu") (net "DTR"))
 (segment (start 91.47229 91.717573) (end 91.47229 85.77229) (width 0.2) (layer "B.Cu") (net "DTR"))
 (segment (start 88.571991 101.197274) (end 89.631991 101.197274) (width 0.2) (layer "B.Cu") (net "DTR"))
 (segment (start 86.291991 101.197274) (end 88.571991 101.197274) (width 0.2) (layer "B.Cu") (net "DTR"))
 (segment (start 96.55229 85.77229) (end 100.017274 89.237274) (width 0.2) (layer "F.Cu") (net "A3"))
 (segment (start 100.017274 89.237274) (end 106.891991 89.237274) (width 0.2) (layer "F.Cu") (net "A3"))
 (segment (start 107.791991 90.137274) (end 107.791991 90.737274) (width 0.2) (layer "F.Cu") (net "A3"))
 (segment (start 106.891991 89.237274) (end 107.791991 90.137274) (width 0.2) (layer "F.Cu") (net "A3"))
 (segment (start 108.591991 90.137274) (end 108.591991 90.737274) (width 0.2) (layer "F.Cu") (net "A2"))
 (segment (start 107.291991 88.837274) (end 108.591991 90.137274) (width 0.2) (layer "F.Cu") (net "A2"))
 (segment (start 102.157274 88.837274) (end 107.291991 88.837274) (width 0.2) (layer "F.Cu") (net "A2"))
 (segment (start 99.09229 85.77229) (end 102.157274 88.837274) (width 0.2) (layer "F.Cu") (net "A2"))
 (segment (start 110.091991 91.071588) (end 110.091991 92.237274) (width 0.2) (layer "F.Cu") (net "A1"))
 (segment (start 107.457677 88.437274) (end 110.091991 91.071588) (width 0.2) (layer "F.Cu") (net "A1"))
 (segment (start 104.277274 88.437274) (end 107.457677 88.437274) (width 0.2) (layer "F.Cu") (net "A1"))
 (segment (start 101.61229 85.77229) (end 104.277274 88.437274) (width 0.2) (layer "F.Cu") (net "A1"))
 (segment (start 104.15229 85.77229) (end 106.417274 88.037274) (width 0.2) (layer "F.Cu") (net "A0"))
 (segment (start 110.791991 92.937274) (end 110.691991 93.037274) (width 0.2) (layer "F.Cu") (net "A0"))
 (segment (start 110.691991 93.037274) (end 110.091991 93.037274) (width 0.2) (layer "F.Cu") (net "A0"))
 (segment (start 110.791991 91.205902) (end 110.791991 92.937274) (width 0.2) (layer "F.Cu") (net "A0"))
 (segment (start 107.623363 88.037274) (end 110.791991 91.205902) (width 0.2) (layer "F.Cu") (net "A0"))
 (segment (start 106.417274 88.037274) (end 107.623363 88.037274) (width 0.2) (layer "F.Cu") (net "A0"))
 (segment (start 112.42771 91.50771) (end 112.42771 97.305811) (width 0.2) (layer "F.Cu") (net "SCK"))
 (segment (start 106.69229 85.77229) (end 112.42771 91.50771) (width 0.2) (layer "F.Cu") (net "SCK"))
 (segment (start 111.896247 97.837274) (end 110.091991 97.837274) (width 0.2) (layer "F.Cu") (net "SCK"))
 (segment (start 112.42771 97.305811) (end 111.896247 97.837274) (width 0.2) (layer "F.Cu") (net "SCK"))
 (via (at 91.791991 98.037274) (size 0.55) (drill 0.15) (layers "F.Cu" "B.Cu") (capping no) (covering (front no) (back no))
  (plugging (front no) (back no)) (filling no) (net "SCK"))
 (segment (start 106.69229 90.636975) (end 105.023252 92.306013) (width 0.2) (layer "B.Cu") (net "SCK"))
 (segment (start 106.69229 85.77229) (end 106.69229 90.636975) (width 0.2) (layer "B.Cu") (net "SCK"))
 (segment (start 105.023252 92.306013) (end 97.523252 92.306013) (width 0.2) (layer "B.Cu") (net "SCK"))
 (segment (start 97.523252 92.306013) (end 91.791991 98.037274) (width 0.2) (layer "B.Cu") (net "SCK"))
 (segment (start 110.961933 99.337274) (end 108.591991 99.337274) (width 0.2) (layer "F.Cu") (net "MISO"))
 (segment (start 109.23229 85.77229) (end 112.82771 89.36771) (width 0.2) (layer "F.Cu") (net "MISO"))
 (segment (start 112.82771 89.36771) (end 112.82771 97.471497) (width 0.2) (layer "F.Cu") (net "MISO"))
 (segment (start 112.82771 97.471497) (end 110.961933 99.337274) (width 0.2) (layer "F.Cu") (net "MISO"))
 (segment (start 113.22771 87.22771) (end 111.77229 85.77229) (width 0.2) (layer "F.Cu") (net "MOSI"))
 (segment (start 107.791991 99.337274) (end 107.791991 99.762274) (width 0.2) (layer "F.Cu") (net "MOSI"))
 (segment (start 108.066991 100.037274) (end 110.827619 100.037274) (width 0.2) (layer "F.Cu") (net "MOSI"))
 (segment (start 107.791991 99.762274) (end 108.066991 100.037274) (width 0.2) (layer "F.Cu") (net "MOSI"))
 (segment (start 113.22771 97.637183) (end 113.22771 87.22771) (width 0.2) (layer "F.Cu") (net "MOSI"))
 (segment (start 110.827619 100.037274) (end 113.22771 97.637183) (width 0.2) (layer "F.Cu") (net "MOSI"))
 (segment (start 110.893304 100.537274) (end 107.791991 100.537274) (width 0.2) (layer "F.Cu") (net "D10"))
 (segment (start 106.991991 99.737274) (end 106.991991 99.337274) (width 0.2) (layer "F.Cu") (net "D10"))
 (segment (start 114.31229 85.77229) (end 114.31229 97.118288) (width 0.2) (layer "F.Cu") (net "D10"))
 (segment (start 107.791991 100.537274) (end 106.991991 99.737274) (width 0.2) (layer "F.Cu") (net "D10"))
 (segment (start 114.31229 97.118288) (end 110.893304 100.537274) (width 0.2) (layer "F.Cu") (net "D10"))
 (segment (start 100.391991 92.737274) (end 100.891991 92.237274) (width 0.2) (layer "F.Cu") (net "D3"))
 (segment (start 100.891991 92.237274) (end 101.491991 92.237274) (width 0.2) (layer "F.Cu") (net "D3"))
 (segment (start 99.031991 104.037274) (end 100.391991 102.677274) (width 0.2) (layer "F.Cu") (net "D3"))
 (segment (start 100.391991 102.677274) (end 100.391991 92.737274) (width 0.2) (layer "F.Cu") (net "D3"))
 (segment (start 101.066991 93.037274) (end 100.791991 93.312274) (width 0.2) (layer "F.Cu") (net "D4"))
 (segment (start 100.791991 93.312274) (end 100.791991 103.277274) (width 0.2) (layer "F.Cu") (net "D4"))
 (segment (start 100.791991 103.277274) (end 101.551991 104.037274) (width 0.2) (layer "F.Cu") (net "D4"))
 (segment (start 101.491991 93.037274) (end 101.066991 93.037274) (width 0.2) (layer "F.Cu") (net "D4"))
 (via (at 97.475768 97.587736) (size 0.55) (drill 0.15) (layers "F.Cu" "B.Cu") (capping no) (covering (front no) (back no))
  (plugging (front no) (back no)) (filling no) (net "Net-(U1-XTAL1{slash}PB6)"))
 (via (at 101.491991 97.037274) (size 0.55) (drill 0.15) (layers "F.Cu" "B.Cu") (capping no) (covering (front no) (back no))
  (plugging (front no) (back no)) (filling no) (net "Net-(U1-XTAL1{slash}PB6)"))
 (segment (start 98.08991 97.037274) (end 101.491991 97.037274) (width 0.2) (layer "B.Cu") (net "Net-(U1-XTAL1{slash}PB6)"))
 (segment (start 97.475768 97.587736) (end 96.776337 97.587736) (width 0.2) (layer "B.Cu") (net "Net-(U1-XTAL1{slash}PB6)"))
 (segment (start 97.475768 97.587736) (end 97.539448 97.587736) (width 0.2) (layer "B.Cu") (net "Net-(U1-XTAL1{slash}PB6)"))
 (segment (start 96.776337 97.587736) (end 96.633933 97.445332) (width 0.2) (layer "B.Cu") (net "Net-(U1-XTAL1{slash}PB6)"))
 (segment (start 97.539448 97.587736) (end 98.08991 97.037274) (width 0.2) (layer "B.Cu") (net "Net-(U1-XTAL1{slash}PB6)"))
 (via (at 101.491991 97.837274) (size 0.55) (drill 0.15) (layers "F.Cu" "B.Cu") (capping no) (covering (front no) (back no))
  (plugging (front no) (back no)) (filling no) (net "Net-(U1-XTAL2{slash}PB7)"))
 (via (at 97.115214 100.416132) (size 0.55) (drill 0.15) (layers "F.Cu" "B.Cu") (capping no) (covering (front no) (back no))
  (plugging (front no) (back no)) (filling no) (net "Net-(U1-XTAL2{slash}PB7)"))
 (segment (start 96.633933 100.829216) (end 96.70213 100.829216) (width 0.2) (layer "B.Cu") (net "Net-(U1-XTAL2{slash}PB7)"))
 (segment (start 96.70213 100.829216) (end 97.115214 100.416132) (width 0.2) (layer "B.Cu") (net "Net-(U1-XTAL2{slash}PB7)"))
 (segment (start 98.913133 100.416132) (end 97.115214 100.416132) (width 0.2) (layer "B.Cu") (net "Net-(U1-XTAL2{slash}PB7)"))
 (segment (start 101.491991 97.837274) (end 98.913133 100.416132) (width 0.2) (layer "B.Cu") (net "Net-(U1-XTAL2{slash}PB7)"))
 (segment (start 102.991991 102.937274) (end 102.991991 99.337274) (width 0.2) (layer "F.Cu") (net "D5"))
 (segment (start 104.091991 104.037274) (end 102.991991 102.937274) (width 0.2) (layer "F.Cu") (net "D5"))
 (segment (start 103.791991 101.197274) (end 103.791991 99.337274) (width 0.2) (layer "F.Cu") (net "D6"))
 (segment (start 106.631991 104.037274) (end 103.791991 101.197274) (width 0.2) (layer "F.Cu") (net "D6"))
 (segment (start 109.171991 104.037274) (end 108.691991 104.037274) (width 0.2) (layer "F.Cu") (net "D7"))
 (segment (start 108.691991 104.037274) (end 104.591991 99.937274) (width 0.2) (layer "F.Cu") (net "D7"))
 (segment (start 104.591991 99.937274) (end 104.591991 99.337274) (width 0.2) (layer "F.Cu") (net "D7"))
 (segment (start 105.391991 99.70296) (end 105.391991 99.337274) (width 0.2) (layer "F.Cu") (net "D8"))
 (segment (start 111.711991 104.037274) (end 109.611991 101.937274) (width 0.2) (layer "F.Cu") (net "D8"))
 (segment (start 107.626305 101.937274) (end 105.391991 99.70296) (width 0.2) (layer "F.Cu") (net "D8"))
 (segment (start 109.611991 101.937274) (end 107.626305 101.937274) (width 0.2) (layer "F.Cu") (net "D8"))
 (segment (start 111.751991 101.537274) (end 107.791991 101.537274) (width 0.2) (layer "F.Cu") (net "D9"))
 (segment (start 106.191991 99.937274) (end 107.791991 101.537274) (width 0.2) (layer "F.Cu") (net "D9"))
 (segment (start 114.251991 104.037274) (end 111.751991 101.537274) (width 0.2) (layer "F.Cu") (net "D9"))
 (segment (start 106.191991 99.337274) (end 106.191991 99.937274) (width 0.2) (layer "F.Cu") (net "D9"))
 (segment (start 111.495653 95.437274) (end 111.67771 95.619331) (width 0.2) (layer "F.Cu") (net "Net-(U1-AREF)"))
 (segment (start 110.091991 95.437274) (end 111.495653 95.437274) (width 0.2) (layer "F.Cu") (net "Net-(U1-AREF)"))
 (segment (start 104.591991 90.312274) (end 104.316991 90.037274) (width 0.2) (layer "F.Cu") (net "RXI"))
 (segment (start 88.871991 104.037274) (end 88.871991 98.697274) (width 0.2) (layer "F.Cu") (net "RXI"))
 (segment (start 92.371991 90.037274) (end 86.291991 96.117274) (width 0.2) (layer "F.Cu") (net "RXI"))
 (segment (start 88.871991 98.697274) (end 86.291991 96.117274) (width 0.2) (layer "F.Cu") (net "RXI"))
 (segment (start 104.591991 90.737274) (end 104.591991 90.312274) (width 0.2) (layer "F.Cu") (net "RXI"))
 (segment (start 104.316991 90.037274) (end 92.371991 90.037274) (width 0.2) (layer "F.Cu") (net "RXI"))
 (via (at 103.791991 90.737274) (size 0.55) (drill 0.15) (layers "F.Cu" "B.Cu") (capping no) (covering (front no) (back no))
  (plugging (front no) (back no)) (filling no) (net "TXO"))
 (segment (start 86.291991 98.657274) (end 85.141991 99.807274) (width 0.2) (layer "B.Cu") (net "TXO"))
 (segment (start 103.791991 90.737274) (end 103.591991 90.737274) (width 0.2) (layer "B.Cu") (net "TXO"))
 (segment (start 93.411991 91.537274) (end 102.791991 91.537274) (width 0.2) (layer "B.Cu") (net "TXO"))
 (segment (start 103.591991 90.737274) (end 102.791991 91.537274) (width 0.2) (layer "B.Cu") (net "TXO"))
 (segment (start 85.141991 99.807274) (end 85.141991 102.847274) (width 0.2) (layer "B.Cu") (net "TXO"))
 (segment (start 85.141991 102.847274) (end 86.331991 104.037274) (width 0.2) (layer "B.Cu") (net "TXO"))
 (segment (start 86.291991 98.657274) (end 93.411991 91.537274) (width 0.2) (layer "B.Cu") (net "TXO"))
 (segment (start 99.991991 92.512274) (end 101.766991 90.737274) (width 0.2) (layer "F.Cu") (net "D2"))
 (segment (start 99.991991 100.537274) (end 99.991991 92.512274) (width 0.2) (layer "F.Cu") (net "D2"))
 (segment (start 101.766991 90.737274) (end 102.991991 90.737274) (width 0.2) (layer "F.Cu") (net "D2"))
 (segment (start 96.491991 104.037274) (end 99.991991 100.537274) (width 0.2) (layer "F.Cu") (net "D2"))
 (segment (start 88.291991 91.387274) (end 89.46289 91.387274) (width 0.2) (layer "F.Cu") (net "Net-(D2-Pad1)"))
 (segment (start 89.46289 91.387274) (end 89.592463 91.516847) (width 0.2) (layer "F.Cu") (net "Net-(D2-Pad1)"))
 (segment (start 95.291991 92.312274) (end 96.941991 92.312274) (width 0.2) (layer "F.Cu") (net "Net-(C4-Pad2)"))
 (segment (start 96.941991 92.312274) (end 97.666991 93.037274) (width 0.2) (layer "F.Cu") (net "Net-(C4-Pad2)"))
 (segment (start 91.791991 99.09092) (end 91.77998 99.078909) (width 0.2) (layer "F.Cu") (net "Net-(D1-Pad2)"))
 (segment (start 91.791991 99.983627) (end 91.791991 99.09092) (width 0.2) (layer "F.Cu") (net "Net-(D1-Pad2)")))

